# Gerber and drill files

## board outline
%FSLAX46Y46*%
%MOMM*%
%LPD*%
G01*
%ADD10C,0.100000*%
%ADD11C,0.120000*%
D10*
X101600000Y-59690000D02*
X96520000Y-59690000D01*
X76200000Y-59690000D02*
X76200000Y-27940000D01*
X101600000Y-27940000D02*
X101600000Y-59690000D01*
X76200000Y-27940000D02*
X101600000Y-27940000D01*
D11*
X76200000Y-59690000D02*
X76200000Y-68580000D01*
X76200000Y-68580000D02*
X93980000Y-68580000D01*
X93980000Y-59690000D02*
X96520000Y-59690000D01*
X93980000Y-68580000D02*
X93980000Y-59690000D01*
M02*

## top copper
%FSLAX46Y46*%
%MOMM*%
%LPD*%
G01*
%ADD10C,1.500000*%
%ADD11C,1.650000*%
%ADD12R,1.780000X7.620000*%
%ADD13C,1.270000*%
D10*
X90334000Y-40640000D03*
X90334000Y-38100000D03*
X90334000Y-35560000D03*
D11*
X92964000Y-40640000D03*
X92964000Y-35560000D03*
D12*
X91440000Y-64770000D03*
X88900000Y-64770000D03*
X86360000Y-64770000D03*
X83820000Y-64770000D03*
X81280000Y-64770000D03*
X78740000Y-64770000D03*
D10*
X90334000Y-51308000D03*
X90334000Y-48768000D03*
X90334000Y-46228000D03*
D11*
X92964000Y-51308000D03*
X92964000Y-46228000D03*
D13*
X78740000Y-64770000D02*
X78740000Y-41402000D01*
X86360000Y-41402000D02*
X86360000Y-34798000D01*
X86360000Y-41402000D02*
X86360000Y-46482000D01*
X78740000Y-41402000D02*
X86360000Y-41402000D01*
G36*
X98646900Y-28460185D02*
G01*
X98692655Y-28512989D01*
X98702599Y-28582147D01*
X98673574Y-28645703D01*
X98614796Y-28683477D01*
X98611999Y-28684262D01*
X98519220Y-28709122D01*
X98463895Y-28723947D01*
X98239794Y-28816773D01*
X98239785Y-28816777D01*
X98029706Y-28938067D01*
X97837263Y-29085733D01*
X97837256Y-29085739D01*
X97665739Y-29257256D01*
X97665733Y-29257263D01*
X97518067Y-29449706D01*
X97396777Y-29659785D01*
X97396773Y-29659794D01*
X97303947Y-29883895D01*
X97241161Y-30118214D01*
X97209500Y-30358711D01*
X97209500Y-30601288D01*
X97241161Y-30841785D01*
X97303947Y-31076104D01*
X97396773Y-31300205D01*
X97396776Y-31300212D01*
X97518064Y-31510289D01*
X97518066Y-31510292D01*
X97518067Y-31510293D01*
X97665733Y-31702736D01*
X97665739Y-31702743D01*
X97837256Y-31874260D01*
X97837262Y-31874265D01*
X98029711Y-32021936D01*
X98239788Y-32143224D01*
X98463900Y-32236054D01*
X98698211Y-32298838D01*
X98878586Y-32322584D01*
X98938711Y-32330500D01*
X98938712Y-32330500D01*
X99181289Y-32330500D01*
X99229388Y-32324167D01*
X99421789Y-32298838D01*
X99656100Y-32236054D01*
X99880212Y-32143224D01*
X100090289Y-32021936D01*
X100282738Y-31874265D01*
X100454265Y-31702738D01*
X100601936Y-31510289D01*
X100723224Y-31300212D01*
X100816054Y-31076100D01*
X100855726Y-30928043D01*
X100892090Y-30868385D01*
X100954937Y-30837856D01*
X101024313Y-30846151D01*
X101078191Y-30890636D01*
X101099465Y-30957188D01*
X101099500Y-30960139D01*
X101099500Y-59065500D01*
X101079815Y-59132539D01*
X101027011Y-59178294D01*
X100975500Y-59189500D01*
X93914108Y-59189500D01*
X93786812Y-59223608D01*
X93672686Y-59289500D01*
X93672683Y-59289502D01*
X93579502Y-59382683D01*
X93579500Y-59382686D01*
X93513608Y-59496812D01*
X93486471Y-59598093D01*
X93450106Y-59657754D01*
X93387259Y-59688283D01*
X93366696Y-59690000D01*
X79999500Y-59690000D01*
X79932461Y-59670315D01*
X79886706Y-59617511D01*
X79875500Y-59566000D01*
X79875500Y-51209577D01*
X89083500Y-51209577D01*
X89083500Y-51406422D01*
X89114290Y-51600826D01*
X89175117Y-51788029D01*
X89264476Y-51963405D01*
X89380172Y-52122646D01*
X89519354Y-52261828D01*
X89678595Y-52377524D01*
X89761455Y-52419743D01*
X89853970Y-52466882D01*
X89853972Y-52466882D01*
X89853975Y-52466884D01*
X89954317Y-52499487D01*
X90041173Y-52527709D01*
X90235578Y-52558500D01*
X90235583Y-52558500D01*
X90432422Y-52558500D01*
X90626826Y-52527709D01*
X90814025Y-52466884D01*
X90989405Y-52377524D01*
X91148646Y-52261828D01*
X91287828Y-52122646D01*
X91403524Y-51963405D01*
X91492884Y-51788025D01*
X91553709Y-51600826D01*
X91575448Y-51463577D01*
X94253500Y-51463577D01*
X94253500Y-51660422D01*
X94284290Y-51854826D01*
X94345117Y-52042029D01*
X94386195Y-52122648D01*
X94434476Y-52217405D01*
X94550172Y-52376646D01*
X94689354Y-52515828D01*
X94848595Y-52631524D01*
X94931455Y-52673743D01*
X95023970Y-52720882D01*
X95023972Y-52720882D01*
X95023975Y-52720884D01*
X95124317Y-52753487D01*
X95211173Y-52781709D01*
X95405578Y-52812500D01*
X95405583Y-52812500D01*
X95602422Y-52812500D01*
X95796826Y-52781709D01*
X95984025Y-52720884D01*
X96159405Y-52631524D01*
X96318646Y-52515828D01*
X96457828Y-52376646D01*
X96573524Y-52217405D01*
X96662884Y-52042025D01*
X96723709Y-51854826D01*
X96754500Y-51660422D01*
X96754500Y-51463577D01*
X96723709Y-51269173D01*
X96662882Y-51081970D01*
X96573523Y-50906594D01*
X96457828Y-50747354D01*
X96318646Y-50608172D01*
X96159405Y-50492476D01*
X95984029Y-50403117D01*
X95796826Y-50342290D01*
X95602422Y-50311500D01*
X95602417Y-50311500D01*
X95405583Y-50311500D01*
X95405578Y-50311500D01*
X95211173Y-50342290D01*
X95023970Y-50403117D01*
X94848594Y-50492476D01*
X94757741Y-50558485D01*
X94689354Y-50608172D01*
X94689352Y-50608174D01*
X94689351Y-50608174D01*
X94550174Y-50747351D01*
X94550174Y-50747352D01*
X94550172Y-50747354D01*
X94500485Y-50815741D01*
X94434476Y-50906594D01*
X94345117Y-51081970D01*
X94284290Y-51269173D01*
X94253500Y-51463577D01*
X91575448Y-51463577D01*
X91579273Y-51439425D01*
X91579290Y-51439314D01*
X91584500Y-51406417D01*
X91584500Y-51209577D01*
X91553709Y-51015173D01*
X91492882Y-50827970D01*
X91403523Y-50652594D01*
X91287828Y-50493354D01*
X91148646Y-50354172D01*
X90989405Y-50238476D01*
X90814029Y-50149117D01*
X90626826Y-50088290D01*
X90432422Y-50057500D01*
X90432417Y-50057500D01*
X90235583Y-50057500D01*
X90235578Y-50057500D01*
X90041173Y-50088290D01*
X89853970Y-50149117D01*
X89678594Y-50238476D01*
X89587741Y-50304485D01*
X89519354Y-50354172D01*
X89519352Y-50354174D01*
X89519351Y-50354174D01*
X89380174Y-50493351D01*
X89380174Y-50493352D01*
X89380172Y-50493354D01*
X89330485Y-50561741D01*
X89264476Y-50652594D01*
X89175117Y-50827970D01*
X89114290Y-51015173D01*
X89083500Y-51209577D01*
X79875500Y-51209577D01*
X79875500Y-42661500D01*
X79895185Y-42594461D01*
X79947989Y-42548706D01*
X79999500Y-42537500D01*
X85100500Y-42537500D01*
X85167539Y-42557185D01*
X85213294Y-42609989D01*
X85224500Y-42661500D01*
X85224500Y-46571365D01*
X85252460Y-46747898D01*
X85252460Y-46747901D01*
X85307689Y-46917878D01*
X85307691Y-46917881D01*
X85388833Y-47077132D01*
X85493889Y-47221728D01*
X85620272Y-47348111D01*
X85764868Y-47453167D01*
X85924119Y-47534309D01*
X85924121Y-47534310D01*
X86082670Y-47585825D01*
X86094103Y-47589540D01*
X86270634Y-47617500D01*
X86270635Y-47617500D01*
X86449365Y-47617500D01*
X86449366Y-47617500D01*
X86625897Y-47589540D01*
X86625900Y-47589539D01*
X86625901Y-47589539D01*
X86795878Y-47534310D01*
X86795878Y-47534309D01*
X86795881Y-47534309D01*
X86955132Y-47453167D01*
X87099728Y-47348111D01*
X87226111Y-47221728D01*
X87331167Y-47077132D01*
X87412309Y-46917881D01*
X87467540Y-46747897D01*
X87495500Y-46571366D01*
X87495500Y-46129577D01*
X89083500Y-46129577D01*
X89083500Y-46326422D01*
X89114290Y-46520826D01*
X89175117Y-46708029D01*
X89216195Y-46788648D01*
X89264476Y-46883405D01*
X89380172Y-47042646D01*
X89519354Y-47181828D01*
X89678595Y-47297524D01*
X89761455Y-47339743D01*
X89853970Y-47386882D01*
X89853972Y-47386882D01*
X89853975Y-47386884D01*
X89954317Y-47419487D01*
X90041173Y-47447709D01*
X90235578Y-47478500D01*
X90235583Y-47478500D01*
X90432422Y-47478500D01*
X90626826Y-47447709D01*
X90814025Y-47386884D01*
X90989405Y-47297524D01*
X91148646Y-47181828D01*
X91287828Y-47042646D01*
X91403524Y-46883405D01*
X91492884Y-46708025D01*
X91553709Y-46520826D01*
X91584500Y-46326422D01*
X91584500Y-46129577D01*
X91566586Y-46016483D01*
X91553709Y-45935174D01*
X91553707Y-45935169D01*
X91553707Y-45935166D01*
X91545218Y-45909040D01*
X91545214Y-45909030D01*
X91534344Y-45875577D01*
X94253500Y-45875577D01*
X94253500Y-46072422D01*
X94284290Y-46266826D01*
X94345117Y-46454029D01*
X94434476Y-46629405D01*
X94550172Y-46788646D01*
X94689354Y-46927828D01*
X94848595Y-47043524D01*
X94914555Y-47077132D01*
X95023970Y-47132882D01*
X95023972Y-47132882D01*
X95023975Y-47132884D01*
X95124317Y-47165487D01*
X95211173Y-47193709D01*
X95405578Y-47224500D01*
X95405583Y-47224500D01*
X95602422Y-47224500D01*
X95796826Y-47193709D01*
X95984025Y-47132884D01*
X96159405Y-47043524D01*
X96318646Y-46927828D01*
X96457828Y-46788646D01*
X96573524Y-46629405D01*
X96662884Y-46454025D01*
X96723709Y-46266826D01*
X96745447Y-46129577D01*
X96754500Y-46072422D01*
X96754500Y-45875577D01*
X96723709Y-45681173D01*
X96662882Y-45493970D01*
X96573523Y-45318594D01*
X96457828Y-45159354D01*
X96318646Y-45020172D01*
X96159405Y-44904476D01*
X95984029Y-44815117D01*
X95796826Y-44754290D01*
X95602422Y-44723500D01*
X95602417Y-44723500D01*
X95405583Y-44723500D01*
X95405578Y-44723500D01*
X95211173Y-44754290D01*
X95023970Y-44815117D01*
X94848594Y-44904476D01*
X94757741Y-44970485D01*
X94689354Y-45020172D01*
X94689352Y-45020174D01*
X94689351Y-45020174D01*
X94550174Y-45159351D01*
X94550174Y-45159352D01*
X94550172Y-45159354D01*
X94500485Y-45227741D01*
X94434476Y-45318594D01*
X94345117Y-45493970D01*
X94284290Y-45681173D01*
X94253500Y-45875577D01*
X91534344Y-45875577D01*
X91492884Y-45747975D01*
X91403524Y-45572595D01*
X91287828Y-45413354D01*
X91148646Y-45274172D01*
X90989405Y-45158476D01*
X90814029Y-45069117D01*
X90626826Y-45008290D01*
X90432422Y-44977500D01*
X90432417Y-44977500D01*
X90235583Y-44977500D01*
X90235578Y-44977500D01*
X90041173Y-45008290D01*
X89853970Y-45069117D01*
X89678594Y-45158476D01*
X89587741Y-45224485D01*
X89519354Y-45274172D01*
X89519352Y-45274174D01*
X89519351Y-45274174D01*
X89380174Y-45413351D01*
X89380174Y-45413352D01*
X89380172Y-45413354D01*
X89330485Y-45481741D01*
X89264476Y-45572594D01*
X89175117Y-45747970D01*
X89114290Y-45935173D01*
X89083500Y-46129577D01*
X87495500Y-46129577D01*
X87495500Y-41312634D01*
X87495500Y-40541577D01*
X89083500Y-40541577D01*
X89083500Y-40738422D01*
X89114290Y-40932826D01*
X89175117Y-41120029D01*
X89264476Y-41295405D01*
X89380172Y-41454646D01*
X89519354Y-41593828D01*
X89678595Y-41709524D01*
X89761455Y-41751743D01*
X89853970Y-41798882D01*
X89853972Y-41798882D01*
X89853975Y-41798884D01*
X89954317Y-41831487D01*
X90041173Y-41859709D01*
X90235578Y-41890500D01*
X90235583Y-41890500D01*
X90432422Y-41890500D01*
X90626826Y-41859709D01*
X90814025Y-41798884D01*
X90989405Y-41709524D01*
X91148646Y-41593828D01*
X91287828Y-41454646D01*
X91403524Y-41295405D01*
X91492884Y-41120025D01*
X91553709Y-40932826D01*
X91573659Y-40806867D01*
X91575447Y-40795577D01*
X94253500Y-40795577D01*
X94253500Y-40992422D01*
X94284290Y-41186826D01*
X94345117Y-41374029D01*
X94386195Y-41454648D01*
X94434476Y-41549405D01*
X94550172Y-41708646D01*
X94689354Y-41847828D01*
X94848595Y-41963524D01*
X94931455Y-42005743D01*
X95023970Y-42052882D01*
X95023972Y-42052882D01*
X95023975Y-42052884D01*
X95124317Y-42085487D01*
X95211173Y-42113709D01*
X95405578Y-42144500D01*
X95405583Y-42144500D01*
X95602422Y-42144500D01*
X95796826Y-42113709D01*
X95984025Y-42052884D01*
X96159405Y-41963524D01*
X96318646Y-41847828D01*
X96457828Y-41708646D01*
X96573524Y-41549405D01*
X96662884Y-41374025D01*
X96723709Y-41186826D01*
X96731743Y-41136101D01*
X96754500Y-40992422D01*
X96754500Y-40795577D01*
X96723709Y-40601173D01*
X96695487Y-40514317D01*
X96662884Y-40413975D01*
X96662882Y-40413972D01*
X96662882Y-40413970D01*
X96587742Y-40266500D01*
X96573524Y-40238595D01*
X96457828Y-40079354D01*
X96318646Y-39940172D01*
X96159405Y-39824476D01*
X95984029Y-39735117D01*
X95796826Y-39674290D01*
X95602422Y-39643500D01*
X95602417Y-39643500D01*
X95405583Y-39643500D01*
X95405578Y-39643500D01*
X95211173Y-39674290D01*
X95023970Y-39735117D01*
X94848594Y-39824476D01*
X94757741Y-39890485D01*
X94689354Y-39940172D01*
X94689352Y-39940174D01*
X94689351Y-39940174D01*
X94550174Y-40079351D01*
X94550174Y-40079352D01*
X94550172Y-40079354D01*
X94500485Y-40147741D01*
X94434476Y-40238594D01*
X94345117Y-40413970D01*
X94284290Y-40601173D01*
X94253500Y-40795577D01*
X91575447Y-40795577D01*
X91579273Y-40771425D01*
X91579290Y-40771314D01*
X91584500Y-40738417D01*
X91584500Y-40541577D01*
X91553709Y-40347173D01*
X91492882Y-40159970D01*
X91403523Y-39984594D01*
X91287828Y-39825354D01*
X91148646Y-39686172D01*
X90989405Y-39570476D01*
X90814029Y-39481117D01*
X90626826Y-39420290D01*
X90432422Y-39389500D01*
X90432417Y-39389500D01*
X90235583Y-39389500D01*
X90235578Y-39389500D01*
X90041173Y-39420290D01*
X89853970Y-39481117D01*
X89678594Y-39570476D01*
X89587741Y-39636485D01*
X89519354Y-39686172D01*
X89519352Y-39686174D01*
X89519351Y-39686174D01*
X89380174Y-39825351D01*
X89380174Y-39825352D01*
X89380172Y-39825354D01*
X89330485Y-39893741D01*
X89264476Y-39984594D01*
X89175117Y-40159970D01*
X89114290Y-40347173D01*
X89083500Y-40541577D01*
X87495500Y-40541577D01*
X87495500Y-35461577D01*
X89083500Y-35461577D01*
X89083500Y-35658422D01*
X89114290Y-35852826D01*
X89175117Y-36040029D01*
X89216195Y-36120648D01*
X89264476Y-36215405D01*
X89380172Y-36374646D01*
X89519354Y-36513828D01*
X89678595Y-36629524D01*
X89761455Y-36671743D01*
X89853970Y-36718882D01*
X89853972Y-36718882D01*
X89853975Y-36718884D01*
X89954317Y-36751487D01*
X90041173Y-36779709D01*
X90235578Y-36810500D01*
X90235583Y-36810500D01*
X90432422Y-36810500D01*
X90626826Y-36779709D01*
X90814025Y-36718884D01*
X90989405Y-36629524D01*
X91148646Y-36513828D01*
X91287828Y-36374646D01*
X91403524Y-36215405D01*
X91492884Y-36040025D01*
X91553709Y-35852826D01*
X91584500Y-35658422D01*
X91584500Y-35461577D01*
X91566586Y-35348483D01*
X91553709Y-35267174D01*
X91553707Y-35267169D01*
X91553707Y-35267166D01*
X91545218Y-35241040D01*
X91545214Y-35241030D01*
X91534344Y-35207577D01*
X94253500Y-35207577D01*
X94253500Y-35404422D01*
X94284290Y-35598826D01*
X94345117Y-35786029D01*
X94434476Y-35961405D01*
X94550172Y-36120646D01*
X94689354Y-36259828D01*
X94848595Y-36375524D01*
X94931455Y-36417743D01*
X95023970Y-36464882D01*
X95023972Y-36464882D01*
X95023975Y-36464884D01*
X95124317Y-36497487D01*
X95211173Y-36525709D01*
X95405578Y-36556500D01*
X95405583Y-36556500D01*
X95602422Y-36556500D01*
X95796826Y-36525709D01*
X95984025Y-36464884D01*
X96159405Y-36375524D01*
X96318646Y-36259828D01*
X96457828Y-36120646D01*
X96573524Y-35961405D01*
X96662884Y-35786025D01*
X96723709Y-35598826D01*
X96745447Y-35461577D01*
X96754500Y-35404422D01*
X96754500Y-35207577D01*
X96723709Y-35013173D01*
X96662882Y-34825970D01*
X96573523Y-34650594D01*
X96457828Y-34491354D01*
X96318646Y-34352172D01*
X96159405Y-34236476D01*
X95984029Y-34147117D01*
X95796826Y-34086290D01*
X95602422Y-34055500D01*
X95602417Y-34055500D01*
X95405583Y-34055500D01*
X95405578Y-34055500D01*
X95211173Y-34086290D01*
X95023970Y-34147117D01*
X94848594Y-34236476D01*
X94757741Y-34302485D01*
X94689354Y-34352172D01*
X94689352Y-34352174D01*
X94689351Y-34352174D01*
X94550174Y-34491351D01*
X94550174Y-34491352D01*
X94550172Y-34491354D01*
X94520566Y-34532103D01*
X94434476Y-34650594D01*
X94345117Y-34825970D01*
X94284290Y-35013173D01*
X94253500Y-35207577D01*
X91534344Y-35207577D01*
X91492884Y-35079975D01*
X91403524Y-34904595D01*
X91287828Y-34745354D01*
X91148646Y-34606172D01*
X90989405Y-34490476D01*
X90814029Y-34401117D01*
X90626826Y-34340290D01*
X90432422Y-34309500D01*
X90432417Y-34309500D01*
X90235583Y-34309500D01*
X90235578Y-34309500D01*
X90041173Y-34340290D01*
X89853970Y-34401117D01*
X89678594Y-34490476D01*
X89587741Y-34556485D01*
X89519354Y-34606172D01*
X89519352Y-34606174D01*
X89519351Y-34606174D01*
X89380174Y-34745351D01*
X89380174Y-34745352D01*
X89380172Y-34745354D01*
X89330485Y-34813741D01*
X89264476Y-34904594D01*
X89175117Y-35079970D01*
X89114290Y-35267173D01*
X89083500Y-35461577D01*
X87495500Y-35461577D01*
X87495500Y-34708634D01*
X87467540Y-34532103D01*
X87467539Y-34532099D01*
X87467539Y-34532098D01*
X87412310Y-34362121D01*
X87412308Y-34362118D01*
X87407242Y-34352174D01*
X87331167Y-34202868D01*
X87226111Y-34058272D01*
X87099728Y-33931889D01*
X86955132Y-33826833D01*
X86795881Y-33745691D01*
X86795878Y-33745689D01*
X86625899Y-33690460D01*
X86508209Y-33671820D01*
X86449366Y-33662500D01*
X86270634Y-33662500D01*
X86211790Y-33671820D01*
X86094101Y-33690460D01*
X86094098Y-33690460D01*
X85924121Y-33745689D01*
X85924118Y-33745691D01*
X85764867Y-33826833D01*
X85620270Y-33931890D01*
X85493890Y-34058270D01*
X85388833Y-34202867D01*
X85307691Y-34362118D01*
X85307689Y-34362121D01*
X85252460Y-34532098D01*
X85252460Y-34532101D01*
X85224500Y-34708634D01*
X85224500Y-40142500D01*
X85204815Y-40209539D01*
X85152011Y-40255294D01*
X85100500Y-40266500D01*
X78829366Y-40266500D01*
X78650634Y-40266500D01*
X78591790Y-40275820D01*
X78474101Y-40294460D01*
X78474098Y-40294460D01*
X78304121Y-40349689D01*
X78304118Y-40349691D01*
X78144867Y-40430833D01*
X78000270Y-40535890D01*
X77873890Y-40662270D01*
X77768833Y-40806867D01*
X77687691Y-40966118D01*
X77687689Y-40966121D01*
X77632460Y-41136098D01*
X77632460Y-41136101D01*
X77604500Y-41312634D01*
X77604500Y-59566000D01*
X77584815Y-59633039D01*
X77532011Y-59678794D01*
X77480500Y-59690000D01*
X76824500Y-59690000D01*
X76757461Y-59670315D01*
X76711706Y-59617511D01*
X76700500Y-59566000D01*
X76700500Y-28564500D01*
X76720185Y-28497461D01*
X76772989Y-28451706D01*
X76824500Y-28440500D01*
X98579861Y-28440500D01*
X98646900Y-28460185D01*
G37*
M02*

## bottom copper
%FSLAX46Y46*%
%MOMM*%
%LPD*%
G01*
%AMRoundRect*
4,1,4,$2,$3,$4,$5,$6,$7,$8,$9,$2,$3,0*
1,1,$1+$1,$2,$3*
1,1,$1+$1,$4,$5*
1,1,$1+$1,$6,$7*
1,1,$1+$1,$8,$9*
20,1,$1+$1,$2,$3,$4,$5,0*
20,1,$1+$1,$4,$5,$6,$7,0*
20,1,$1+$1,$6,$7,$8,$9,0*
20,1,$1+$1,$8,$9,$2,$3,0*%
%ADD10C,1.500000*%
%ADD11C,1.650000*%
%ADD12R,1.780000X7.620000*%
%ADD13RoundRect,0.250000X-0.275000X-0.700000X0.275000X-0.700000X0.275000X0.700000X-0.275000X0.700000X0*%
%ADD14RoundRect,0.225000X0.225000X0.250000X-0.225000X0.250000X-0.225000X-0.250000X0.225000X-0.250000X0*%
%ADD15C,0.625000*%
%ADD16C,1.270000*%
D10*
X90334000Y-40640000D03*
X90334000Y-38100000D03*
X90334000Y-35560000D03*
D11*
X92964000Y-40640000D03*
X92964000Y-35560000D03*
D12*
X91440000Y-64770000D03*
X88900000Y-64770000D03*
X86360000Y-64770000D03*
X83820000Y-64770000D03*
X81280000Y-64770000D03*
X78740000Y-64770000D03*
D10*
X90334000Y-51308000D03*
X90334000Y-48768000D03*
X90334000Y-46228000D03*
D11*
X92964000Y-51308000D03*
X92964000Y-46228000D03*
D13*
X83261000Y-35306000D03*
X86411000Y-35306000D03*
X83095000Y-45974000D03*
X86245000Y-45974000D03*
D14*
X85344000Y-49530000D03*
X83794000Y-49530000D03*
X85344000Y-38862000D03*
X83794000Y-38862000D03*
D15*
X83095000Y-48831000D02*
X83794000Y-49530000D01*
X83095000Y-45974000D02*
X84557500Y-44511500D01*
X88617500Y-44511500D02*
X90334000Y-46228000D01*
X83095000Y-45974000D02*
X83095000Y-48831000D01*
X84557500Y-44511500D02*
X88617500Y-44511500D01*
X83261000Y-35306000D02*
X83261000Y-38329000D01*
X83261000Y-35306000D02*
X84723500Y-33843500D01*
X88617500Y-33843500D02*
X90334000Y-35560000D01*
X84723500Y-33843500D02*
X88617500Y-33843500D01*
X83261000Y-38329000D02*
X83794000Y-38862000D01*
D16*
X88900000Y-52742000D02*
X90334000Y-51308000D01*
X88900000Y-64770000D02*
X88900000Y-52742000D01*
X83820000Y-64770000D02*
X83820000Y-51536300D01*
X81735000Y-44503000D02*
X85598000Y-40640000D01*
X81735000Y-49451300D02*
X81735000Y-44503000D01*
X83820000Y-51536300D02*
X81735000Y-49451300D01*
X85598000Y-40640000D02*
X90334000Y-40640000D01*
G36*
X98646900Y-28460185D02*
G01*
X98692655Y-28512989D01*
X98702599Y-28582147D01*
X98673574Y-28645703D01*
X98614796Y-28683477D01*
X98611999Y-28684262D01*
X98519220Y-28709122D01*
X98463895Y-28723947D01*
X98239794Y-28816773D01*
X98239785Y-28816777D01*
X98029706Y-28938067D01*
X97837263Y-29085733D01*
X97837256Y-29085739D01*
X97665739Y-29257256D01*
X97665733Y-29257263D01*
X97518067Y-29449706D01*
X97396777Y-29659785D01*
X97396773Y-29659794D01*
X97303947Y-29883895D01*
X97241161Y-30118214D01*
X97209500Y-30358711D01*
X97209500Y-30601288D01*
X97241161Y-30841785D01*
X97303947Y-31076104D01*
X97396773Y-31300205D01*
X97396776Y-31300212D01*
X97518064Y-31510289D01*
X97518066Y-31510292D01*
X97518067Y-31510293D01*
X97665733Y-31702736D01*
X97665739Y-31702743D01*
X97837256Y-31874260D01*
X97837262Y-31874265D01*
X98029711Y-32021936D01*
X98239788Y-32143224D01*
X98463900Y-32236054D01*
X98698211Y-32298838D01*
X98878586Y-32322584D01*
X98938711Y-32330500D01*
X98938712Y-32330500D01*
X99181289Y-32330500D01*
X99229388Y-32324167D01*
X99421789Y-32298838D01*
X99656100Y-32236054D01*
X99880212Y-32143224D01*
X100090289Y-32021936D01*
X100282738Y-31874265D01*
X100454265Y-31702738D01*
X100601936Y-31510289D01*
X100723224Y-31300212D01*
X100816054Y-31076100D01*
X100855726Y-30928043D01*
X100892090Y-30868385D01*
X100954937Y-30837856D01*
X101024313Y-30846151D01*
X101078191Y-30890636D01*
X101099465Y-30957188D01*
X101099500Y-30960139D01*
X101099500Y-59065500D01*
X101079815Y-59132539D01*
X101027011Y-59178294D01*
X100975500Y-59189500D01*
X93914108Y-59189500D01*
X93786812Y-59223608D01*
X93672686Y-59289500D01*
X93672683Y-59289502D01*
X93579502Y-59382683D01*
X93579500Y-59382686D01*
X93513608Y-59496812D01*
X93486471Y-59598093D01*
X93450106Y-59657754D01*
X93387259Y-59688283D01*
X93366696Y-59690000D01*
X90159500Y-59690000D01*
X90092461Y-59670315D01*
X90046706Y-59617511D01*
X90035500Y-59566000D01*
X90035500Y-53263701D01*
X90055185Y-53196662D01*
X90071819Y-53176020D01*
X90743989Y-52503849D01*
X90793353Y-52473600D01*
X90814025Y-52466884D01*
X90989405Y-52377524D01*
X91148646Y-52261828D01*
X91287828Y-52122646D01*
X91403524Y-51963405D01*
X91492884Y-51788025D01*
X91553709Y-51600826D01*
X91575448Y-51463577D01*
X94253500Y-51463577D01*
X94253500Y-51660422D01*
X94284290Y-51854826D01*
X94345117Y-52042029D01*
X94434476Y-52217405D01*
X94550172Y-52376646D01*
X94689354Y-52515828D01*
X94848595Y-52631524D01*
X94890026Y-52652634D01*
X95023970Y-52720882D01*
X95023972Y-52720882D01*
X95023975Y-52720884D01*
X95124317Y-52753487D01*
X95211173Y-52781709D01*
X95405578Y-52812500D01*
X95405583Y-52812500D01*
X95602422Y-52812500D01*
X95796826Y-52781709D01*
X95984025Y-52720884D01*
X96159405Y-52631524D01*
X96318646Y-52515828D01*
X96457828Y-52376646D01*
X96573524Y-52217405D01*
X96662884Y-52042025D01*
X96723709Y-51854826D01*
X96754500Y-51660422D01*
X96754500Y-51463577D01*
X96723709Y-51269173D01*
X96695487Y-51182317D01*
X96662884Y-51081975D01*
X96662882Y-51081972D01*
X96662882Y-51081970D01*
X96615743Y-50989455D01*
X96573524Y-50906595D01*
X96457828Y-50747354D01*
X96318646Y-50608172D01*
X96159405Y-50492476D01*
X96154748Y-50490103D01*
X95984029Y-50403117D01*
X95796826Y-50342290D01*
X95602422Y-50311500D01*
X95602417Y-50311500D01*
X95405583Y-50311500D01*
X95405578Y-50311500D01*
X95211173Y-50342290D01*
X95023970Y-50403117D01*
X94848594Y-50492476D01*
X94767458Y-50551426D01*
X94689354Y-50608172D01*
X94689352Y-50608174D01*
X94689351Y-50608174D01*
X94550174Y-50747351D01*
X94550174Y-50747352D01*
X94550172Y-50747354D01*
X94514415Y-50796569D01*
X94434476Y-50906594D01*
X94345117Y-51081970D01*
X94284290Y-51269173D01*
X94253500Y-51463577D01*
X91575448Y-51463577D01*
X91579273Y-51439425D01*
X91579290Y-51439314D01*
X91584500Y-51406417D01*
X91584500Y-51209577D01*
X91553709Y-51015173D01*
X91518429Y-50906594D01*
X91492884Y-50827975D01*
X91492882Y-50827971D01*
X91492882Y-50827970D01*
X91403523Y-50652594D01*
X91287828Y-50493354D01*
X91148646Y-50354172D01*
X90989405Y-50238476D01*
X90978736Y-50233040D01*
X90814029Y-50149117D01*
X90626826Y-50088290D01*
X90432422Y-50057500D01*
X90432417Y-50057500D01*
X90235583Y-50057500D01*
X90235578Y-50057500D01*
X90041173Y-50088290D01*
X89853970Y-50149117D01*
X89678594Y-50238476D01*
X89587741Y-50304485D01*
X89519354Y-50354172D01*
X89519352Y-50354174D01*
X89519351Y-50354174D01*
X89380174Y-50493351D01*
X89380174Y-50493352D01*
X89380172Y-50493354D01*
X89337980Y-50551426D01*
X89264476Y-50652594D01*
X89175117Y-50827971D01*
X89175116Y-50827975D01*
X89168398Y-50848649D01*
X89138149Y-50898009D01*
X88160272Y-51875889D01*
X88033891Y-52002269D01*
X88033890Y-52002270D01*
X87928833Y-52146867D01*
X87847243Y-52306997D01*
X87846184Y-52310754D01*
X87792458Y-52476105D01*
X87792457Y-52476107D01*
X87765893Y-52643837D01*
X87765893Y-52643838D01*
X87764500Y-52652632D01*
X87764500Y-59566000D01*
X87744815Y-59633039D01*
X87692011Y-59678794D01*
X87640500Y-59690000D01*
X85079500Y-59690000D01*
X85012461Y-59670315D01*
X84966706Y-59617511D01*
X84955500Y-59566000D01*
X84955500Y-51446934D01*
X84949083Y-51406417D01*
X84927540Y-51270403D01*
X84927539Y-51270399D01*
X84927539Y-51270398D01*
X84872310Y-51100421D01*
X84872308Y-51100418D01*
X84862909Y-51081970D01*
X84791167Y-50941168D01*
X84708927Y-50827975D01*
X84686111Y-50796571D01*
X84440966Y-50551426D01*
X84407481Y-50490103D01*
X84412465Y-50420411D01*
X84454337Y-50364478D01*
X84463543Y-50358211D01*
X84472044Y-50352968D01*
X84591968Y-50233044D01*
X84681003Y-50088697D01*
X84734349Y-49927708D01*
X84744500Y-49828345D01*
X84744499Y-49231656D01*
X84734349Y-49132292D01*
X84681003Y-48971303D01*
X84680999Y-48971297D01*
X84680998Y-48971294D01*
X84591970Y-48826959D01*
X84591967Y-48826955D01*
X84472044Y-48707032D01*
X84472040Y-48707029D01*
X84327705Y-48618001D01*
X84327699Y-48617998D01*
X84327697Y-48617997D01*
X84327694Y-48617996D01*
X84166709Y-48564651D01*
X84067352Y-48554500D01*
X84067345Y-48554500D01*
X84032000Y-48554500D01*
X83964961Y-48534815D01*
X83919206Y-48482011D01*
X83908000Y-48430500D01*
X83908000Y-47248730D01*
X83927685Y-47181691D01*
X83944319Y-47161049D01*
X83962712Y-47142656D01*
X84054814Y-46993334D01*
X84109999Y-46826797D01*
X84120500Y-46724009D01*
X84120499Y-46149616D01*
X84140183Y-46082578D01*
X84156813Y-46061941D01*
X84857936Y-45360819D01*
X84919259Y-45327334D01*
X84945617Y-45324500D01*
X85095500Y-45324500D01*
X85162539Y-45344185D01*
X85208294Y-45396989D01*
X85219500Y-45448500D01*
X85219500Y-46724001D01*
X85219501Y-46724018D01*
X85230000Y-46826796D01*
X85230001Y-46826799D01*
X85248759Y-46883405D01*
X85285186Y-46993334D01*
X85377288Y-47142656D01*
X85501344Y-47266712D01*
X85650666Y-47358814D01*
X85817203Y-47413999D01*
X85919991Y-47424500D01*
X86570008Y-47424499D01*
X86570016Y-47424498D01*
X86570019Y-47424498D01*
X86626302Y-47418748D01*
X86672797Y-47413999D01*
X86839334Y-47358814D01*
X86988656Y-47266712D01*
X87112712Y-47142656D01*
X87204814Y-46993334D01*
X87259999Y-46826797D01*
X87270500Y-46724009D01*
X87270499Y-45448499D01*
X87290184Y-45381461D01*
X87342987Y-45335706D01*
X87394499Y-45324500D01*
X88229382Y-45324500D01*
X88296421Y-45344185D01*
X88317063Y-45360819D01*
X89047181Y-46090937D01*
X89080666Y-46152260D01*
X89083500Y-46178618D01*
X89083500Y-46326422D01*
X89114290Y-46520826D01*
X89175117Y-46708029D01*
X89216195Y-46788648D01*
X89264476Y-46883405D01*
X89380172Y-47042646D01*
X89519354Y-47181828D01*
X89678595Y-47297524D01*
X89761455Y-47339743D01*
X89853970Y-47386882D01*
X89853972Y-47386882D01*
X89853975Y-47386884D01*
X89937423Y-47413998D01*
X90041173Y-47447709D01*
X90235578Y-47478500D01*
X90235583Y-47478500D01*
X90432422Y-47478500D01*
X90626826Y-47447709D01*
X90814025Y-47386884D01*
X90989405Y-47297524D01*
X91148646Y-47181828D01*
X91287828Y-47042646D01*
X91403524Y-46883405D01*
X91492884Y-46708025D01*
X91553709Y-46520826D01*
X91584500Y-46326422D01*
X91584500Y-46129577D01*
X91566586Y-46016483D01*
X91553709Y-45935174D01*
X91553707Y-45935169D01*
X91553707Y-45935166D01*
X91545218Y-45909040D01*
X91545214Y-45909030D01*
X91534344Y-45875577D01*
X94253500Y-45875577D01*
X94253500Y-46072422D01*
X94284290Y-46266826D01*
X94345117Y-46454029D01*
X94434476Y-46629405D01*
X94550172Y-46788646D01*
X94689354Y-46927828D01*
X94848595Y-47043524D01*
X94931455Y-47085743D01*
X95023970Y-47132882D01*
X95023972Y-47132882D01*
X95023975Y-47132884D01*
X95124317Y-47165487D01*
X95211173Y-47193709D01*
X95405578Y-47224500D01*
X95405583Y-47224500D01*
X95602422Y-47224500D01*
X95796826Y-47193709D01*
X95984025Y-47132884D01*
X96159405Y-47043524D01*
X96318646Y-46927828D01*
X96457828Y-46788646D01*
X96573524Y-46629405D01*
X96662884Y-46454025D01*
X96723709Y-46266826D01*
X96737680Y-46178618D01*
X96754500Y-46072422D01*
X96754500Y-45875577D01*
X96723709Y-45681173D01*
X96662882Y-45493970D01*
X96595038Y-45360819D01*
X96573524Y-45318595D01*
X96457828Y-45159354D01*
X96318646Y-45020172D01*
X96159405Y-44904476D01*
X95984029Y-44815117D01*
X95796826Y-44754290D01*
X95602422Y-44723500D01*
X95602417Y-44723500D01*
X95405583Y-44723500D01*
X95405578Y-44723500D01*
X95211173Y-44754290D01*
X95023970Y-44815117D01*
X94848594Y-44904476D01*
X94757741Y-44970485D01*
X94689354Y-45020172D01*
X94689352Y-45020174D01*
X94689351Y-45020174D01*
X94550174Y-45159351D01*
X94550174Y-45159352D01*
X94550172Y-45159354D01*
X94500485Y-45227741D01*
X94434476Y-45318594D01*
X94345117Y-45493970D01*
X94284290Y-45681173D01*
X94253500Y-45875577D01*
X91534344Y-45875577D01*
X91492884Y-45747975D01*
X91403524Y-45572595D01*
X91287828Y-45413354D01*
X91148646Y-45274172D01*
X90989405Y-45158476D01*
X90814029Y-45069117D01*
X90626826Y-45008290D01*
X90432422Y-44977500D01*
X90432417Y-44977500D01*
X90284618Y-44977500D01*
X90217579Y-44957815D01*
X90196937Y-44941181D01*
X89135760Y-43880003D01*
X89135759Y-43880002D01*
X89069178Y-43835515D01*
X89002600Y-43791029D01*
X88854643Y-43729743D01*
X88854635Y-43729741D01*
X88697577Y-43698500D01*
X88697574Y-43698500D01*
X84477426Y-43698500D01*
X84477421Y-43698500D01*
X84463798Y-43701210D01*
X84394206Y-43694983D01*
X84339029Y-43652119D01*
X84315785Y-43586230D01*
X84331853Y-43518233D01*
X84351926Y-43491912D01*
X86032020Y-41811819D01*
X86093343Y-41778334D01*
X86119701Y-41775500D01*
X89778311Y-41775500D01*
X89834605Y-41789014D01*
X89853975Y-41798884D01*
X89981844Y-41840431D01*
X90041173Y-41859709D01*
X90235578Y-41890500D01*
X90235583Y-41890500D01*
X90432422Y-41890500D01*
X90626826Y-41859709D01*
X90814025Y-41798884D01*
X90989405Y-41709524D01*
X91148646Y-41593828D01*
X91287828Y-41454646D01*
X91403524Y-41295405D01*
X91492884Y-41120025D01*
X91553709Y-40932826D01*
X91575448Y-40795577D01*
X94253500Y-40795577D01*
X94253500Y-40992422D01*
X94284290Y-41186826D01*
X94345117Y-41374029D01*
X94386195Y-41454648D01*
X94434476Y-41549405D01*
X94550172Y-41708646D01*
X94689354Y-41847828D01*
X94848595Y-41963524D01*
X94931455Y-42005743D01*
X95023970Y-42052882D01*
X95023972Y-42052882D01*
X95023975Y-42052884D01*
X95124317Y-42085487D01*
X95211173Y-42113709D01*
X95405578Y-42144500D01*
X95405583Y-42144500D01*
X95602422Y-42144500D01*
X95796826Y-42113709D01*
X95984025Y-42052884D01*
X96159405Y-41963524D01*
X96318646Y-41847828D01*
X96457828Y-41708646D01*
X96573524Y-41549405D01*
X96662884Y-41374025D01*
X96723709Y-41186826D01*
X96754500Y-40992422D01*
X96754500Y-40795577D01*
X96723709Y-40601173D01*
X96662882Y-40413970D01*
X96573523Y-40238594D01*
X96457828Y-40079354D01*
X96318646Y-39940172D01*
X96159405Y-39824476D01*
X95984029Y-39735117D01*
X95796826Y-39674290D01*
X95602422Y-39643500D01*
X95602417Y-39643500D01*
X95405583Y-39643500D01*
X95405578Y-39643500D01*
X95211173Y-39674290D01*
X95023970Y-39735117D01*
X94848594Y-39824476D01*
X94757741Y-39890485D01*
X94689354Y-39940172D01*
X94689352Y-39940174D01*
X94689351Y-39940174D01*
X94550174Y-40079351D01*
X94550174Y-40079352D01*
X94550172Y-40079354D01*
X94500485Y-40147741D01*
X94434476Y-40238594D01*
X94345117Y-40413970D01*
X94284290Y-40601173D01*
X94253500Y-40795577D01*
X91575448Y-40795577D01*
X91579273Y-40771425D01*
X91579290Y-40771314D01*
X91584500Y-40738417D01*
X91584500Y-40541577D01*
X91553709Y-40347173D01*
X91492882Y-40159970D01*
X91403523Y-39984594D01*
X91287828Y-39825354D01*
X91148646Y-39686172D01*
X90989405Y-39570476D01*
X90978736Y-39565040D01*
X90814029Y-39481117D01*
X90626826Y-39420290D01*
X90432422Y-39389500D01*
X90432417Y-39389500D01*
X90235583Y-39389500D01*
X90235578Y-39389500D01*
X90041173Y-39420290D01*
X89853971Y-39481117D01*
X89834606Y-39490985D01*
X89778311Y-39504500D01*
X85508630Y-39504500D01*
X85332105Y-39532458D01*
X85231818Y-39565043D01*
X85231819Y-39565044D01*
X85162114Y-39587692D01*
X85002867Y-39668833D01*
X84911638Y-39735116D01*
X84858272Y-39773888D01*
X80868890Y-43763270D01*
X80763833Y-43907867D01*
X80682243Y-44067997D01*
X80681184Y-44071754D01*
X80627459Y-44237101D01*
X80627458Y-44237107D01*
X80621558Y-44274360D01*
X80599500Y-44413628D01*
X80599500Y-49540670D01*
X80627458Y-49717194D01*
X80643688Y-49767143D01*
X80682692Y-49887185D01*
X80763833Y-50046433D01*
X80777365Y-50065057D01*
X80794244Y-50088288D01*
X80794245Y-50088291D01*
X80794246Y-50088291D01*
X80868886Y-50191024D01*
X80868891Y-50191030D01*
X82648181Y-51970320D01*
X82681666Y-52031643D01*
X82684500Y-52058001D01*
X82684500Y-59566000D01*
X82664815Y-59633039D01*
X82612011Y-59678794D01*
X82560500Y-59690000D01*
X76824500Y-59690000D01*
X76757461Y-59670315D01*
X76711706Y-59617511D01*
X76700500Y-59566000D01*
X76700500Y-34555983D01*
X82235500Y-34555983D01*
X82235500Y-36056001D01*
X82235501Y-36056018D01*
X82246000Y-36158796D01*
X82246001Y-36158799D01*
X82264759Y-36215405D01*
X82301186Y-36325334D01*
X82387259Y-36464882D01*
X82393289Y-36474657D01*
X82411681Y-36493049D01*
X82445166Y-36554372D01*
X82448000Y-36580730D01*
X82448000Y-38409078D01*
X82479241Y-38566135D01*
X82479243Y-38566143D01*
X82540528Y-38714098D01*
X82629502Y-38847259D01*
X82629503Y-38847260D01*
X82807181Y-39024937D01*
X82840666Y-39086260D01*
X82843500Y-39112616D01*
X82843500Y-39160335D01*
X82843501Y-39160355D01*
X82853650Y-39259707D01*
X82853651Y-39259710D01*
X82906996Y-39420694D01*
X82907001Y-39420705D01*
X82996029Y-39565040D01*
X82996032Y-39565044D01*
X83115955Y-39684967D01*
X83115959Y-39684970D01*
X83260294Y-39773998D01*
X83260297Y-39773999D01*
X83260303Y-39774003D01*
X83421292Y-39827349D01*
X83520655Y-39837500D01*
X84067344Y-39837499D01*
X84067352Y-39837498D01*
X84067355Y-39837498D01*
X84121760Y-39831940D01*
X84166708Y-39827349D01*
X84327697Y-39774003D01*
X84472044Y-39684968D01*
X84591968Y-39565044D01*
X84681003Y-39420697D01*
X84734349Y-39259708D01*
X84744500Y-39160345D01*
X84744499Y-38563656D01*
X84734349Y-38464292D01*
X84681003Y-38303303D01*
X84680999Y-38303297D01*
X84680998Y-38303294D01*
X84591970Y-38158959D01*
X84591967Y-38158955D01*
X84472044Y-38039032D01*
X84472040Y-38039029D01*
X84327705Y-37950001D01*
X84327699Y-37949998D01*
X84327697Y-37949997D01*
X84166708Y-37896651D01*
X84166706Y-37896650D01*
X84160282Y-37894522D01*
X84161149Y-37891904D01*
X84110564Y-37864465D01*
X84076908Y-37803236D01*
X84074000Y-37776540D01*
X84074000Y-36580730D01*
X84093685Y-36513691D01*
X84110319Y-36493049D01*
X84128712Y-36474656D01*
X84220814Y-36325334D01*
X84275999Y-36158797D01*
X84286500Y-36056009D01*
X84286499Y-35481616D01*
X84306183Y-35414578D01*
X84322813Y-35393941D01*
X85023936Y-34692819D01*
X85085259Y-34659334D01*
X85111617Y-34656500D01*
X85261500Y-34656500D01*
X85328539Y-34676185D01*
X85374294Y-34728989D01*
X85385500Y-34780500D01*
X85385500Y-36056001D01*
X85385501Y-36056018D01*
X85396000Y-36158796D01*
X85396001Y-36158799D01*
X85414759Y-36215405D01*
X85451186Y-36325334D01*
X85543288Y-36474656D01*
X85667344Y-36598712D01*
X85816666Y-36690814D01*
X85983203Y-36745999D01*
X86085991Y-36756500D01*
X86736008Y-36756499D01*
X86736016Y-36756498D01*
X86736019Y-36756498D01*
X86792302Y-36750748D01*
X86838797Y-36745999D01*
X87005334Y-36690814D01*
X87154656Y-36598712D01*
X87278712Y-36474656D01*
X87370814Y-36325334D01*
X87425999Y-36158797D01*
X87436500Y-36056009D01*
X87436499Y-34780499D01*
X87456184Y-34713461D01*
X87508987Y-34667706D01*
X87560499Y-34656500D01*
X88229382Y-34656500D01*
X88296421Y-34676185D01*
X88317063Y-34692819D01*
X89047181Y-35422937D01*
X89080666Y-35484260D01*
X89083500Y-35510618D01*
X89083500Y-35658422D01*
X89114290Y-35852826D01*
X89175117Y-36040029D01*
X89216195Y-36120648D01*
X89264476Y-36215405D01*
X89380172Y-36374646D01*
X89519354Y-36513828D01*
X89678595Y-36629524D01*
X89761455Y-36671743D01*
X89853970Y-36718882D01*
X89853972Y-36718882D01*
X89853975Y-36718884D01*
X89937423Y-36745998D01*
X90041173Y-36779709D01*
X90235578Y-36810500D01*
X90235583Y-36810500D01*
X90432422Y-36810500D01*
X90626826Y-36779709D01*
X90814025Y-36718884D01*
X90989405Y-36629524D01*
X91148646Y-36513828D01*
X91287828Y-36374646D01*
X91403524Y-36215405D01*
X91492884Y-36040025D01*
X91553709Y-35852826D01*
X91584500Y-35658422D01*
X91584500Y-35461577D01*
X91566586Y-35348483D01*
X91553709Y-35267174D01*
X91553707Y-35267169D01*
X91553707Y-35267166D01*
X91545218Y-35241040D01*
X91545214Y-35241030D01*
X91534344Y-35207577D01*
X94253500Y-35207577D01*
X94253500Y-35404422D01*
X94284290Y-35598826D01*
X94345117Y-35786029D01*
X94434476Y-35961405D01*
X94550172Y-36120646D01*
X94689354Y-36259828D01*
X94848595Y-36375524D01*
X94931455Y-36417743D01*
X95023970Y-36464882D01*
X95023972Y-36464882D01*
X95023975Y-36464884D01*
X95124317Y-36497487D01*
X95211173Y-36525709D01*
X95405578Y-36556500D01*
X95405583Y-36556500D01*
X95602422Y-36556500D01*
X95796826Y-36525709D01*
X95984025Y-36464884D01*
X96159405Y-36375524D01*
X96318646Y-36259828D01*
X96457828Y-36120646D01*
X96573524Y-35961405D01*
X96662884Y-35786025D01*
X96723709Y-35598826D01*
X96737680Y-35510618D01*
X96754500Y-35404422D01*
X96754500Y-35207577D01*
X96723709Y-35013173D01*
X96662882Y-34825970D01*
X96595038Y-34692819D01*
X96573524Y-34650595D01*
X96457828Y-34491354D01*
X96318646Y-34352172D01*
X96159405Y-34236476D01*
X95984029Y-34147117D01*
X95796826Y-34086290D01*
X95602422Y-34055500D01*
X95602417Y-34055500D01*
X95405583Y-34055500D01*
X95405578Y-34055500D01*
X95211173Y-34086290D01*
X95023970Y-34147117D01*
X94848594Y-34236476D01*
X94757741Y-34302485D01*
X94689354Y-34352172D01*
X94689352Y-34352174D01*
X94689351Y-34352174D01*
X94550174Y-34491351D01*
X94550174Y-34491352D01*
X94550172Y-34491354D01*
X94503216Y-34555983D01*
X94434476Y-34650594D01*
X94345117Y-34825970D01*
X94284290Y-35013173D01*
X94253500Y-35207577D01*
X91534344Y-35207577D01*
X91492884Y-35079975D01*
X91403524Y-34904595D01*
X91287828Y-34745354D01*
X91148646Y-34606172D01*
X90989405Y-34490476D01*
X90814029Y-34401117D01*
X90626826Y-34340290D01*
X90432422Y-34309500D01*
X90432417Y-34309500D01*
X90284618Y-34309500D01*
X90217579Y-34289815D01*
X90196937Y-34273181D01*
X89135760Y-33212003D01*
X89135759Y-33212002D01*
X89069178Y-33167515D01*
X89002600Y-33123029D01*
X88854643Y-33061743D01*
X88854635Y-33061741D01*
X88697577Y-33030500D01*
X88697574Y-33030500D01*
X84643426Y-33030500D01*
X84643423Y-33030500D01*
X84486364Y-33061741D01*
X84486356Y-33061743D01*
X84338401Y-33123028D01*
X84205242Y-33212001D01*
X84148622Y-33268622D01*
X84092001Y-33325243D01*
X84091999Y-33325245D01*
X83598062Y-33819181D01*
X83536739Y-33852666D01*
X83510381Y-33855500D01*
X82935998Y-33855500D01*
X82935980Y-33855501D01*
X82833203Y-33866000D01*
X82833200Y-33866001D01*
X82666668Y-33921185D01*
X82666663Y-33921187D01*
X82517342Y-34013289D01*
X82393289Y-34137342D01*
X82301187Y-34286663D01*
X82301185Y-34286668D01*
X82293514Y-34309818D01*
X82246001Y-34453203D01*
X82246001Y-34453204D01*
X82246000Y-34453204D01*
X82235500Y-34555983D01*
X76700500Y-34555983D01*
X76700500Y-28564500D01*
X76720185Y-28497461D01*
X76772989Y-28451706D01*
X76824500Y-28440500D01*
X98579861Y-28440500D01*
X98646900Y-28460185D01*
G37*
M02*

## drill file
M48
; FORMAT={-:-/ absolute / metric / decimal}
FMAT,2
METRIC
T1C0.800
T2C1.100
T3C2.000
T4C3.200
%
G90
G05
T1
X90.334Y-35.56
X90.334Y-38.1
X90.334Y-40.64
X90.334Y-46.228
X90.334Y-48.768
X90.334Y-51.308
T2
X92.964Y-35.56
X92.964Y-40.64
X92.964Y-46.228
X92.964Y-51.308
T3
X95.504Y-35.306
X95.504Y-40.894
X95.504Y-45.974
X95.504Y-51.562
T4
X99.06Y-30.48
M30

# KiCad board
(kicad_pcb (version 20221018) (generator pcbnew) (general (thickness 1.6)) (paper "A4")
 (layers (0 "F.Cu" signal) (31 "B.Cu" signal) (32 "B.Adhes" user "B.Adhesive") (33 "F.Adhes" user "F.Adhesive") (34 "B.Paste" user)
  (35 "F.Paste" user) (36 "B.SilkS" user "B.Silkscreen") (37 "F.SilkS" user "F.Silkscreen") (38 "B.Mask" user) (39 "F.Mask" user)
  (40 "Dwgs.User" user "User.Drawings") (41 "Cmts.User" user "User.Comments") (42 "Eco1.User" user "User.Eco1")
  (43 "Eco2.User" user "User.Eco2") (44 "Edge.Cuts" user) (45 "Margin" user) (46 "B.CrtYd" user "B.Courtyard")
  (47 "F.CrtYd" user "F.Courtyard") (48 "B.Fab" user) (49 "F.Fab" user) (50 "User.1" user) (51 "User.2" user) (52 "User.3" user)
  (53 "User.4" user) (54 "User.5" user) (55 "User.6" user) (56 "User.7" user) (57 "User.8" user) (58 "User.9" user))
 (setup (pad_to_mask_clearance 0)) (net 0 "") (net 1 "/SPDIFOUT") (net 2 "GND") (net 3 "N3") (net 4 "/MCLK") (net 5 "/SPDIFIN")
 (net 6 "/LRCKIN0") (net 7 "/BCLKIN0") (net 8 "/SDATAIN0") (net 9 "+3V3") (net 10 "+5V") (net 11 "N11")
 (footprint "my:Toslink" (layer "F.Cu") (at 92.964 38.1 -90) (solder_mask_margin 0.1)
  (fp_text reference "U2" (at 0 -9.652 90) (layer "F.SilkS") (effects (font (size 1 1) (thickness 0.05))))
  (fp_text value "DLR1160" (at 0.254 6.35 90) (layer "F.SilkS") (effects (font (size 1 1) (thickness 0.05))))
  (pad "" np_thru_hole circle (at -2.794 -2.54 270) (size 2 2) (drill 2) (layers "*.Cu" "*.Mask"))
  (pad "" np_thru_hole circle (at 2.794 -2.54 270) (size 2 2) (drill 2) (layers "*.Cu" "*.Mask"))
  (pad "1" thru_hole circle (at 2.54 2.63 270) (size 1.5 1.5) (drill 0.8) (layers "*.Cu" "*.Mask" "F.SilkS") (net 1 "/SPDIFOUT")
   (solder_mask_margin 0.2))
  (pad "2" thru_hole circle (at 0 2.63 270) (size 1.5 1.5) (drill 0.8) (layers "*.Cu" "*.Mask" "F.SilkS") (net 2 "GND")
   (solder_mask_margin 0.2))
  (pad "3" thru_hole circle (at -2.54 2.63 270) (size 1.5 1.5) (drill 0.8) (layers "*.Cu" "*.Mask" "F.SilkS") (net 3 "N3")
   (solder_mask_margin 0.2))
  (pad "NC1" thru_hole circle (at 2.54 0 270) (size 1.65 1.65) (drill 1.1) (layers "*.Cu" "*.Mask" "F.SilkS") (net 2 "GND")
   (solder_mask_margin 0.2))
  (pad "NC2" thru_hole circle (at -2.54 0 270) (size 1.65 1.65) (drill 1.1) (layers "*.Cu" "*.Mask" "F.SilkS") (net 2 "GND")
   (solder_mask_margin 0.2)))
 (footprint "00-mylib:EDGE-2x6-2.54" (layer "F.Cu") (at 85.09 64.77)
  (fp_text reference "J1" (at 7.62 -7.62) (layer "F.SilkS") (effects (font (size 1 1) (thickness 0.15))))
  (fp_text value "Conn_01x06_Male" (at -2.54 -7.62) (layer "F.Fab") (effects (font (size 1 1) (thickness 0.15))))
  (fp_line (start -8.89 -5.08) (end -8.89 3.81) (stroke (width 0.12) (type default)) (layer "Edge.Cuts"))
  (fp_line (start -8.89 3.81) (end 8.89 3.81) (stroke (width 0.12) (type default)) (layer "Edge.Cuts"))
  (fp_line (start 8.89 -5.08) (end 11.43 -5.08) (stroke (width 0.12) (type default)) (layer "Edge.Cuts"))
  (fp_line (start 8.89 3.81) (end 8.89 -5.08) (stroke (width 0.12) (type default)) (layer "Edge.Cuts"))
  (pad "1" connect rect (at 6.35 0) (size 1.78 7.62) (layers "F.Cu" "F.Mask") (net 2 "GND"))
  (pad "2" connect rect (at 6.35 0) (size 1.78 7.62) (layers "B.Cu" "B.Mask") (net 2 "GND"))
  (pad "3" connect rect (at 3.81 0) (size 1.78 7.62) (layers "F.Cu" "F.Mask") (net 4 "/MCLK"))
  (pad "4" connect rect (at 3.81 0) (size 1.78 7.62) (layers "B.Cu" "B.Mask") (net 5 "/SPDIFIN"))
  (pad "5" connect rect (at 1.27 0) (size 1.78 7.62) (layers "F.Cu" "F.Mask") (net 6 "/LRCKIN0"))
  (pad "6" connect rect (at 1.27 0) (size 1.78 7.62) (layers "B.Cu" "B.Mask") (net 2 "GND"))
  (pad "7" connect rect (at -1.27 0) (size 1.78 7.62) (layers "F.Cu" "F.Mask") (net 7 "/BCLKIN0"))
  (pad "8" connect rect (at -1.27 0) (size 1.78 7.62) (layers "B.Cu" "B.Mask") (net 1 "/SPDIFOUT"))
  (pad "9" connect rect (at -3.81 0) (size 1.78 7.62) (layers "F.Cu" "F.Mask") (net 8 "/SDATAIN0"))
  (pad "10" connect rect (at -3.81 0) (size 1.78 7.62) (layers "B.Cu" "B.Mask") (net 2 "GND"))
  (pad "11" connect rect (at -6.35 0) (size 1.78 7.62) (layers "F.Cu" "F.Mask") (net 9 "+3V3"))
  (pad "12" connect rect (at -6.35 0) (size 1.78 7.62) (layers "B.Cu" "B.Mask") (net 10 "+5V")))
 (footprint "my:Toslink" (layer "F.Cu") (at 92.964 48.768 -90) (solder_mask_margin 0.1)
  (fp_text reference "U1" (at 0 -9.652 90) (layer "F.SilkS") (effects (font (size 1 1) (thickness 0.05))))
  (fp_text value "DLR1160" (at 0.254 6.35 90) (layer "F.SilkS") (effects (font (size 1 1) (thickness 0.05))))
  (pad "" np_thru_hole circle (at -2.794 -2.54 270) (size 2 2) (drill 2) (layers "*.Cu" "*.Mask"))
  (pad "" np_thru_hole circle (at 2.794 -2.54 270) (size 2 2) (drill 2) (layers "*.Cu" "*.Mask"))
  (pad "1" thru_hole circle (at 2.54 2.63 270) (size 1.5 1.5) (drill 0.8) (layers "*.Cu" "*.Mask" "F.SilkS") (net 5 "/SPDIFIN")
   (solder_mask_margin 0.2))
  (pad "2" thru_hole circle (at 0 2.63 270) (size 1.5 1.5) (drill 0.8) (layers "*.Cu" "*.Mask" "F.SilkS") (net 2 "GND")
   (solder_mask_margin 0.2))
  (pad "3" thru_hole circle (at -2.54 2.63 270) (size 1.5 1.5) (drill 0.8) (layers "*.Cu" "*.Mask" "F.SilkS") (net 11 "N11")
   (solder_mask_margin 0.2))
  (pad "NC1" thru_hole circle (at 2.54 0 270) (size 1.65 1.65) (drill 1.1) (layers "*.Cu" "*.Mask" "F.SilkS") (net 2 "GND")
   (solder_mask_margin 0.2))
  (pad "NC2" thru_hole circle (at -2.54 0 270) (size 1.65 1.65) (drill 1.1) (layers "*.Cu" "*.Mask" "F.SilkS") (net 2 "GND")
   (solder_mask_margin 0.2)))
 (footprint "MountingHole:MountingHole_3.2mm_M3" (layer "F.Cu") (at 99.06 30.48)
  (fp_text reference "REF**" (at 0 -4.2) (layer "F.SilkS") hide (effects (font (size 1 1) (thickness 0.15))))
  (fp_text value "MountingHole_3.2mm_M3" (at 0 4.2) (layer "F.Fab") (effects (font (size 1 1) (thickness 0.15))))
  (pad "" np_thru_hole circle (at 0 0) (size 3.2 3.2) (drill 3.2) (layers "F&B.Cu" "*.Mask")))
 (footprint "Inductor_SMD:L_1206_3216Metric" (layer "B.Cu") (at 84.836 35.306)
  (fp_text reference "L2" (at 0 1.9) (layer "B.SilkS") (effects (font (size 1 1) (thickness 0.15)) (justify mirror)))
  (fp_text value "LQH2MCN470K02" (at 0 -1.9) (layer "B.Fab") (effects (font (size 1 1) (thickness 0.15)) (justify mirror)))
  (pad "1" smd roundrect (at -1.575 0) (size 1.05 1.9) (layers "B.Cu" "B.Paste" "B.Mask") (roundrect_rratio 0.238095) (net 3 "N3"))
  (pad "2" smd roundrect (at 1.575 0) (size 1.05 1.9) (layers "B.Cu" "B.Paste" "B.Mask") (roundrect_rratio 0.238095) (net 9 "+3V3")))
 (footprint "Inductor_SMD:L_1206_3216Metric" (layer "B.Cu") (at 84.67 45.974)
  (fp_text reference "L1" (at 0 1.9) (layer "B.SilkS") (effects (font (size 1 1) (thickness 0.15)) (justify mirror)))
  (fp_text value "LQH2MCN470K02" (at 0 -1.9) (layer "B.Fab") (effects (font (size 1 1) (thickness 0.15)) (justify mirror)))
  (pad "1" smd roundrect (at -1.575 0) (size 1.05 1.9) (layers "B.Cu" "B.Paste" "B.Mask") (roundrect_rratio 0.238095) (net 11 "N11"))
  (pad "2" smd roundrect (at 1.575 0) (size 1.05 1.9) (layers "B.Cu" "B.Paste" "B.Mask") (roundrect_rratio 0.238095) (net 9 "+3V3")))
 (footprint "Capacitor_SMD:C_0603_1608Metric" (layer "B.Cu") (at 84.569 49.53 180)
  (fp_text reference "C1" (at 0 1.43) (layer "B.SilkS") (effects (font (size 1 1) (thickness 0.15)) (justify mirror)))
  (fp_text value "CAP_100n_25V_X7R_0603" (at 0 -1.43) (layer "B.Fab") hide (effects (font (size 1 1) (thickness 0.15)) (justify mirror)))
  (pad "1" smd roundrect (at -0.775 0 180) (size 0.9 0.95) (layers "B.Cu" "B.Paste" "B.Mask") (roundrect_rratio 0.25) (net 2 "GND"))
  (pad "2" smd roundrect (at 0.775 0 180) (size 0.9 0.95) (layers "B.Cu" "B.Paste" "B.Mask") (roundrect_rratio 0.25) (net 11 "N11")))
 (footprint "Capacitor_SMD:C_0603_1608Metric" (layer "B.Cu") (at 84.569 38.862 180)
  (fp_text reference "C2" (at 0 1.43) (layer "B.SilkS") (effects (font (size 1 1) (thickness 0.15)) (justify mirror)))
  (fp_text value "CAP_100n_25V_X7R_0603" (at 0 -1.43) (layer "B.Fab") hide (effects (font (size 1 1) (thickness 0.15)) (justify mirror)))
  (pad "1" smd roundrect (at -0.775 0 180) (size 0.9 0.95) (layers "B.Cu" "B.Paste" "B.Mask") (roundrect_rratio 0.25) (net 2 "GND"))
  (pad "2" smd roundrect (at 0.775 0 180) (size 0.9 0.95) (layers "B.Cu" "B.Paste" "B.Mask") (roundrect_rratio 0.25) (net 3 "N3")))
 (gr_line (start 101.6 59.69) (end 96.52 59.69) (stroke (width 0.1) (type default)) (layer "Edge.Cuts"))
 (gr_line (start 76.2 59.69) (end 76.2 27.94) (stroke (width 0.1) (type default)) (layer "Edge.Cuts"))
 (gr_line (start 101.6 27.94) (end 101.6 59.69) (stroke (width 0.1) (type default)) (layer "Edge.Cuts"))
 (gr_line (start 76.2 27.94) (end 101.6 27.94) (stroke (width 0.1) (type default)) (layer "Edge.Cuts"))
 (segment (start 83.095 48.831) (end 83.794 49.53) (width 0.625) (layer "B.Cu") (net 11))
 (segment (start 83.095 45.974) (end 84.5575 44.5115) (width 0.625) (layer "B.Cu") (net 11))
 (segment (start 88.6175 44.5115) (end 90.334 46.228) (width 0.625) (layer "B.Cu") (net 11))
 (segment (start 83.095 45.974) (end 83.095 48.831) (width 0.625) (layer "B.Cu") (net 11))
 (segment (start 84.5575 44.5115) (end 88.6175 44.5115) (width 0.625) (layer "B.Cu") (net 11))
 (segment (start 83.261 35.306) (end 83.261 38.329) (width 0.625) (layer "B.Cu") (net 3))
 (segment (start 83.261 35.306) (end 84.7235 33.8435) (width 0.625) (layer "B.Cu") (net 3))
 (segment (start 88.6175 33.8435) (end 90.334 35.56) (width 0.625) (layer "B.Cu") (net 3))
 (segment (start 84.7235 33.8435) (end 88.6175 33.8435) (width 0.625) (layer "B.Cu") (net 3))
 (segment (start 83.261 38.329) (end 83.794 38.862) (width 0.625) (layer "B.Cu") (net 3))
 (segment (start 88.9 52.742) (end 90.334 51.308) (width 1.27) (layer "B.Cu") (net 5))
 (segment (start 88.9 64.77) (end 88.9 52.742) (width 1.27) (layer "B.Cu") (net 5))
 (segment (start 83.82 64.77) (end 83.82 51.5363) (width 1.27) (layer "B.Cu") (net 1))
 (segment (start 81.735 44.503) (end 85.598 40.64) (width 1.27) (layer "B.Cu") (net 1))
 (segment (start 81.735 49.4513) (end 81.735 44.503) (width 1.27) (layer "B.Cu") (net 1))
 (segment (start 83.82 51.5363) (end 81.735 49.4513) (width 1.27) (layer "B.Cu") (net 1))
 (segment (start 85.598 40.64) (end 90.334 40.64) (width 1.27) (layer "B.Cu") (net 1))
 (segment (start 78.74 64.77) (end 78.74 41.402) (width 1.27) (layer "F.Cu") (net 9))
 (segment (start 86.36 41.402) (end 86.36 34.798) (width 1.27) (layer "F.Cu") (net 9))
 (segment (start 86.36 41.402) (end 86.36 46.482) (width 1.27) (layer "F.Cu") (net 9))
 (segment (start 78.74 41.402) (end 86.36 41.402) (width 1.27) (layer "F.Cu") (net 9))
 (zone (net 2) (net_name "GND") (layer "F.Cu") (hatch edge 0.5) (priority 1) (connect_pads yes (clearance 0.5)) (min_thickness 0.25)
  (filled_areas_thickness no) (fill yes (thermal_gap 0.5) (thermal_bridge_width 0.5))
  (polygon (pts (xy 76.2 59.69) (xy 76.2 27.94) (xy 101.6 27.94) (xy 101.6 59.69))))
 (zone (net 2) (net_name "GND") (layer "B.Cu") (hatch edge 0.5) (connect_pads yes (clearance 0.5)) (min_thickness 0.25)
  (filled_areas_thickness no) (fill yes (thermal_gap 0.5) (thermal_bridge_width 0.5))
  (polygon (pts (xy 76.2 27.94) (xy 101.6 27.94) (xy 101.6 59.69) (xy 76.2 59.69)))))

